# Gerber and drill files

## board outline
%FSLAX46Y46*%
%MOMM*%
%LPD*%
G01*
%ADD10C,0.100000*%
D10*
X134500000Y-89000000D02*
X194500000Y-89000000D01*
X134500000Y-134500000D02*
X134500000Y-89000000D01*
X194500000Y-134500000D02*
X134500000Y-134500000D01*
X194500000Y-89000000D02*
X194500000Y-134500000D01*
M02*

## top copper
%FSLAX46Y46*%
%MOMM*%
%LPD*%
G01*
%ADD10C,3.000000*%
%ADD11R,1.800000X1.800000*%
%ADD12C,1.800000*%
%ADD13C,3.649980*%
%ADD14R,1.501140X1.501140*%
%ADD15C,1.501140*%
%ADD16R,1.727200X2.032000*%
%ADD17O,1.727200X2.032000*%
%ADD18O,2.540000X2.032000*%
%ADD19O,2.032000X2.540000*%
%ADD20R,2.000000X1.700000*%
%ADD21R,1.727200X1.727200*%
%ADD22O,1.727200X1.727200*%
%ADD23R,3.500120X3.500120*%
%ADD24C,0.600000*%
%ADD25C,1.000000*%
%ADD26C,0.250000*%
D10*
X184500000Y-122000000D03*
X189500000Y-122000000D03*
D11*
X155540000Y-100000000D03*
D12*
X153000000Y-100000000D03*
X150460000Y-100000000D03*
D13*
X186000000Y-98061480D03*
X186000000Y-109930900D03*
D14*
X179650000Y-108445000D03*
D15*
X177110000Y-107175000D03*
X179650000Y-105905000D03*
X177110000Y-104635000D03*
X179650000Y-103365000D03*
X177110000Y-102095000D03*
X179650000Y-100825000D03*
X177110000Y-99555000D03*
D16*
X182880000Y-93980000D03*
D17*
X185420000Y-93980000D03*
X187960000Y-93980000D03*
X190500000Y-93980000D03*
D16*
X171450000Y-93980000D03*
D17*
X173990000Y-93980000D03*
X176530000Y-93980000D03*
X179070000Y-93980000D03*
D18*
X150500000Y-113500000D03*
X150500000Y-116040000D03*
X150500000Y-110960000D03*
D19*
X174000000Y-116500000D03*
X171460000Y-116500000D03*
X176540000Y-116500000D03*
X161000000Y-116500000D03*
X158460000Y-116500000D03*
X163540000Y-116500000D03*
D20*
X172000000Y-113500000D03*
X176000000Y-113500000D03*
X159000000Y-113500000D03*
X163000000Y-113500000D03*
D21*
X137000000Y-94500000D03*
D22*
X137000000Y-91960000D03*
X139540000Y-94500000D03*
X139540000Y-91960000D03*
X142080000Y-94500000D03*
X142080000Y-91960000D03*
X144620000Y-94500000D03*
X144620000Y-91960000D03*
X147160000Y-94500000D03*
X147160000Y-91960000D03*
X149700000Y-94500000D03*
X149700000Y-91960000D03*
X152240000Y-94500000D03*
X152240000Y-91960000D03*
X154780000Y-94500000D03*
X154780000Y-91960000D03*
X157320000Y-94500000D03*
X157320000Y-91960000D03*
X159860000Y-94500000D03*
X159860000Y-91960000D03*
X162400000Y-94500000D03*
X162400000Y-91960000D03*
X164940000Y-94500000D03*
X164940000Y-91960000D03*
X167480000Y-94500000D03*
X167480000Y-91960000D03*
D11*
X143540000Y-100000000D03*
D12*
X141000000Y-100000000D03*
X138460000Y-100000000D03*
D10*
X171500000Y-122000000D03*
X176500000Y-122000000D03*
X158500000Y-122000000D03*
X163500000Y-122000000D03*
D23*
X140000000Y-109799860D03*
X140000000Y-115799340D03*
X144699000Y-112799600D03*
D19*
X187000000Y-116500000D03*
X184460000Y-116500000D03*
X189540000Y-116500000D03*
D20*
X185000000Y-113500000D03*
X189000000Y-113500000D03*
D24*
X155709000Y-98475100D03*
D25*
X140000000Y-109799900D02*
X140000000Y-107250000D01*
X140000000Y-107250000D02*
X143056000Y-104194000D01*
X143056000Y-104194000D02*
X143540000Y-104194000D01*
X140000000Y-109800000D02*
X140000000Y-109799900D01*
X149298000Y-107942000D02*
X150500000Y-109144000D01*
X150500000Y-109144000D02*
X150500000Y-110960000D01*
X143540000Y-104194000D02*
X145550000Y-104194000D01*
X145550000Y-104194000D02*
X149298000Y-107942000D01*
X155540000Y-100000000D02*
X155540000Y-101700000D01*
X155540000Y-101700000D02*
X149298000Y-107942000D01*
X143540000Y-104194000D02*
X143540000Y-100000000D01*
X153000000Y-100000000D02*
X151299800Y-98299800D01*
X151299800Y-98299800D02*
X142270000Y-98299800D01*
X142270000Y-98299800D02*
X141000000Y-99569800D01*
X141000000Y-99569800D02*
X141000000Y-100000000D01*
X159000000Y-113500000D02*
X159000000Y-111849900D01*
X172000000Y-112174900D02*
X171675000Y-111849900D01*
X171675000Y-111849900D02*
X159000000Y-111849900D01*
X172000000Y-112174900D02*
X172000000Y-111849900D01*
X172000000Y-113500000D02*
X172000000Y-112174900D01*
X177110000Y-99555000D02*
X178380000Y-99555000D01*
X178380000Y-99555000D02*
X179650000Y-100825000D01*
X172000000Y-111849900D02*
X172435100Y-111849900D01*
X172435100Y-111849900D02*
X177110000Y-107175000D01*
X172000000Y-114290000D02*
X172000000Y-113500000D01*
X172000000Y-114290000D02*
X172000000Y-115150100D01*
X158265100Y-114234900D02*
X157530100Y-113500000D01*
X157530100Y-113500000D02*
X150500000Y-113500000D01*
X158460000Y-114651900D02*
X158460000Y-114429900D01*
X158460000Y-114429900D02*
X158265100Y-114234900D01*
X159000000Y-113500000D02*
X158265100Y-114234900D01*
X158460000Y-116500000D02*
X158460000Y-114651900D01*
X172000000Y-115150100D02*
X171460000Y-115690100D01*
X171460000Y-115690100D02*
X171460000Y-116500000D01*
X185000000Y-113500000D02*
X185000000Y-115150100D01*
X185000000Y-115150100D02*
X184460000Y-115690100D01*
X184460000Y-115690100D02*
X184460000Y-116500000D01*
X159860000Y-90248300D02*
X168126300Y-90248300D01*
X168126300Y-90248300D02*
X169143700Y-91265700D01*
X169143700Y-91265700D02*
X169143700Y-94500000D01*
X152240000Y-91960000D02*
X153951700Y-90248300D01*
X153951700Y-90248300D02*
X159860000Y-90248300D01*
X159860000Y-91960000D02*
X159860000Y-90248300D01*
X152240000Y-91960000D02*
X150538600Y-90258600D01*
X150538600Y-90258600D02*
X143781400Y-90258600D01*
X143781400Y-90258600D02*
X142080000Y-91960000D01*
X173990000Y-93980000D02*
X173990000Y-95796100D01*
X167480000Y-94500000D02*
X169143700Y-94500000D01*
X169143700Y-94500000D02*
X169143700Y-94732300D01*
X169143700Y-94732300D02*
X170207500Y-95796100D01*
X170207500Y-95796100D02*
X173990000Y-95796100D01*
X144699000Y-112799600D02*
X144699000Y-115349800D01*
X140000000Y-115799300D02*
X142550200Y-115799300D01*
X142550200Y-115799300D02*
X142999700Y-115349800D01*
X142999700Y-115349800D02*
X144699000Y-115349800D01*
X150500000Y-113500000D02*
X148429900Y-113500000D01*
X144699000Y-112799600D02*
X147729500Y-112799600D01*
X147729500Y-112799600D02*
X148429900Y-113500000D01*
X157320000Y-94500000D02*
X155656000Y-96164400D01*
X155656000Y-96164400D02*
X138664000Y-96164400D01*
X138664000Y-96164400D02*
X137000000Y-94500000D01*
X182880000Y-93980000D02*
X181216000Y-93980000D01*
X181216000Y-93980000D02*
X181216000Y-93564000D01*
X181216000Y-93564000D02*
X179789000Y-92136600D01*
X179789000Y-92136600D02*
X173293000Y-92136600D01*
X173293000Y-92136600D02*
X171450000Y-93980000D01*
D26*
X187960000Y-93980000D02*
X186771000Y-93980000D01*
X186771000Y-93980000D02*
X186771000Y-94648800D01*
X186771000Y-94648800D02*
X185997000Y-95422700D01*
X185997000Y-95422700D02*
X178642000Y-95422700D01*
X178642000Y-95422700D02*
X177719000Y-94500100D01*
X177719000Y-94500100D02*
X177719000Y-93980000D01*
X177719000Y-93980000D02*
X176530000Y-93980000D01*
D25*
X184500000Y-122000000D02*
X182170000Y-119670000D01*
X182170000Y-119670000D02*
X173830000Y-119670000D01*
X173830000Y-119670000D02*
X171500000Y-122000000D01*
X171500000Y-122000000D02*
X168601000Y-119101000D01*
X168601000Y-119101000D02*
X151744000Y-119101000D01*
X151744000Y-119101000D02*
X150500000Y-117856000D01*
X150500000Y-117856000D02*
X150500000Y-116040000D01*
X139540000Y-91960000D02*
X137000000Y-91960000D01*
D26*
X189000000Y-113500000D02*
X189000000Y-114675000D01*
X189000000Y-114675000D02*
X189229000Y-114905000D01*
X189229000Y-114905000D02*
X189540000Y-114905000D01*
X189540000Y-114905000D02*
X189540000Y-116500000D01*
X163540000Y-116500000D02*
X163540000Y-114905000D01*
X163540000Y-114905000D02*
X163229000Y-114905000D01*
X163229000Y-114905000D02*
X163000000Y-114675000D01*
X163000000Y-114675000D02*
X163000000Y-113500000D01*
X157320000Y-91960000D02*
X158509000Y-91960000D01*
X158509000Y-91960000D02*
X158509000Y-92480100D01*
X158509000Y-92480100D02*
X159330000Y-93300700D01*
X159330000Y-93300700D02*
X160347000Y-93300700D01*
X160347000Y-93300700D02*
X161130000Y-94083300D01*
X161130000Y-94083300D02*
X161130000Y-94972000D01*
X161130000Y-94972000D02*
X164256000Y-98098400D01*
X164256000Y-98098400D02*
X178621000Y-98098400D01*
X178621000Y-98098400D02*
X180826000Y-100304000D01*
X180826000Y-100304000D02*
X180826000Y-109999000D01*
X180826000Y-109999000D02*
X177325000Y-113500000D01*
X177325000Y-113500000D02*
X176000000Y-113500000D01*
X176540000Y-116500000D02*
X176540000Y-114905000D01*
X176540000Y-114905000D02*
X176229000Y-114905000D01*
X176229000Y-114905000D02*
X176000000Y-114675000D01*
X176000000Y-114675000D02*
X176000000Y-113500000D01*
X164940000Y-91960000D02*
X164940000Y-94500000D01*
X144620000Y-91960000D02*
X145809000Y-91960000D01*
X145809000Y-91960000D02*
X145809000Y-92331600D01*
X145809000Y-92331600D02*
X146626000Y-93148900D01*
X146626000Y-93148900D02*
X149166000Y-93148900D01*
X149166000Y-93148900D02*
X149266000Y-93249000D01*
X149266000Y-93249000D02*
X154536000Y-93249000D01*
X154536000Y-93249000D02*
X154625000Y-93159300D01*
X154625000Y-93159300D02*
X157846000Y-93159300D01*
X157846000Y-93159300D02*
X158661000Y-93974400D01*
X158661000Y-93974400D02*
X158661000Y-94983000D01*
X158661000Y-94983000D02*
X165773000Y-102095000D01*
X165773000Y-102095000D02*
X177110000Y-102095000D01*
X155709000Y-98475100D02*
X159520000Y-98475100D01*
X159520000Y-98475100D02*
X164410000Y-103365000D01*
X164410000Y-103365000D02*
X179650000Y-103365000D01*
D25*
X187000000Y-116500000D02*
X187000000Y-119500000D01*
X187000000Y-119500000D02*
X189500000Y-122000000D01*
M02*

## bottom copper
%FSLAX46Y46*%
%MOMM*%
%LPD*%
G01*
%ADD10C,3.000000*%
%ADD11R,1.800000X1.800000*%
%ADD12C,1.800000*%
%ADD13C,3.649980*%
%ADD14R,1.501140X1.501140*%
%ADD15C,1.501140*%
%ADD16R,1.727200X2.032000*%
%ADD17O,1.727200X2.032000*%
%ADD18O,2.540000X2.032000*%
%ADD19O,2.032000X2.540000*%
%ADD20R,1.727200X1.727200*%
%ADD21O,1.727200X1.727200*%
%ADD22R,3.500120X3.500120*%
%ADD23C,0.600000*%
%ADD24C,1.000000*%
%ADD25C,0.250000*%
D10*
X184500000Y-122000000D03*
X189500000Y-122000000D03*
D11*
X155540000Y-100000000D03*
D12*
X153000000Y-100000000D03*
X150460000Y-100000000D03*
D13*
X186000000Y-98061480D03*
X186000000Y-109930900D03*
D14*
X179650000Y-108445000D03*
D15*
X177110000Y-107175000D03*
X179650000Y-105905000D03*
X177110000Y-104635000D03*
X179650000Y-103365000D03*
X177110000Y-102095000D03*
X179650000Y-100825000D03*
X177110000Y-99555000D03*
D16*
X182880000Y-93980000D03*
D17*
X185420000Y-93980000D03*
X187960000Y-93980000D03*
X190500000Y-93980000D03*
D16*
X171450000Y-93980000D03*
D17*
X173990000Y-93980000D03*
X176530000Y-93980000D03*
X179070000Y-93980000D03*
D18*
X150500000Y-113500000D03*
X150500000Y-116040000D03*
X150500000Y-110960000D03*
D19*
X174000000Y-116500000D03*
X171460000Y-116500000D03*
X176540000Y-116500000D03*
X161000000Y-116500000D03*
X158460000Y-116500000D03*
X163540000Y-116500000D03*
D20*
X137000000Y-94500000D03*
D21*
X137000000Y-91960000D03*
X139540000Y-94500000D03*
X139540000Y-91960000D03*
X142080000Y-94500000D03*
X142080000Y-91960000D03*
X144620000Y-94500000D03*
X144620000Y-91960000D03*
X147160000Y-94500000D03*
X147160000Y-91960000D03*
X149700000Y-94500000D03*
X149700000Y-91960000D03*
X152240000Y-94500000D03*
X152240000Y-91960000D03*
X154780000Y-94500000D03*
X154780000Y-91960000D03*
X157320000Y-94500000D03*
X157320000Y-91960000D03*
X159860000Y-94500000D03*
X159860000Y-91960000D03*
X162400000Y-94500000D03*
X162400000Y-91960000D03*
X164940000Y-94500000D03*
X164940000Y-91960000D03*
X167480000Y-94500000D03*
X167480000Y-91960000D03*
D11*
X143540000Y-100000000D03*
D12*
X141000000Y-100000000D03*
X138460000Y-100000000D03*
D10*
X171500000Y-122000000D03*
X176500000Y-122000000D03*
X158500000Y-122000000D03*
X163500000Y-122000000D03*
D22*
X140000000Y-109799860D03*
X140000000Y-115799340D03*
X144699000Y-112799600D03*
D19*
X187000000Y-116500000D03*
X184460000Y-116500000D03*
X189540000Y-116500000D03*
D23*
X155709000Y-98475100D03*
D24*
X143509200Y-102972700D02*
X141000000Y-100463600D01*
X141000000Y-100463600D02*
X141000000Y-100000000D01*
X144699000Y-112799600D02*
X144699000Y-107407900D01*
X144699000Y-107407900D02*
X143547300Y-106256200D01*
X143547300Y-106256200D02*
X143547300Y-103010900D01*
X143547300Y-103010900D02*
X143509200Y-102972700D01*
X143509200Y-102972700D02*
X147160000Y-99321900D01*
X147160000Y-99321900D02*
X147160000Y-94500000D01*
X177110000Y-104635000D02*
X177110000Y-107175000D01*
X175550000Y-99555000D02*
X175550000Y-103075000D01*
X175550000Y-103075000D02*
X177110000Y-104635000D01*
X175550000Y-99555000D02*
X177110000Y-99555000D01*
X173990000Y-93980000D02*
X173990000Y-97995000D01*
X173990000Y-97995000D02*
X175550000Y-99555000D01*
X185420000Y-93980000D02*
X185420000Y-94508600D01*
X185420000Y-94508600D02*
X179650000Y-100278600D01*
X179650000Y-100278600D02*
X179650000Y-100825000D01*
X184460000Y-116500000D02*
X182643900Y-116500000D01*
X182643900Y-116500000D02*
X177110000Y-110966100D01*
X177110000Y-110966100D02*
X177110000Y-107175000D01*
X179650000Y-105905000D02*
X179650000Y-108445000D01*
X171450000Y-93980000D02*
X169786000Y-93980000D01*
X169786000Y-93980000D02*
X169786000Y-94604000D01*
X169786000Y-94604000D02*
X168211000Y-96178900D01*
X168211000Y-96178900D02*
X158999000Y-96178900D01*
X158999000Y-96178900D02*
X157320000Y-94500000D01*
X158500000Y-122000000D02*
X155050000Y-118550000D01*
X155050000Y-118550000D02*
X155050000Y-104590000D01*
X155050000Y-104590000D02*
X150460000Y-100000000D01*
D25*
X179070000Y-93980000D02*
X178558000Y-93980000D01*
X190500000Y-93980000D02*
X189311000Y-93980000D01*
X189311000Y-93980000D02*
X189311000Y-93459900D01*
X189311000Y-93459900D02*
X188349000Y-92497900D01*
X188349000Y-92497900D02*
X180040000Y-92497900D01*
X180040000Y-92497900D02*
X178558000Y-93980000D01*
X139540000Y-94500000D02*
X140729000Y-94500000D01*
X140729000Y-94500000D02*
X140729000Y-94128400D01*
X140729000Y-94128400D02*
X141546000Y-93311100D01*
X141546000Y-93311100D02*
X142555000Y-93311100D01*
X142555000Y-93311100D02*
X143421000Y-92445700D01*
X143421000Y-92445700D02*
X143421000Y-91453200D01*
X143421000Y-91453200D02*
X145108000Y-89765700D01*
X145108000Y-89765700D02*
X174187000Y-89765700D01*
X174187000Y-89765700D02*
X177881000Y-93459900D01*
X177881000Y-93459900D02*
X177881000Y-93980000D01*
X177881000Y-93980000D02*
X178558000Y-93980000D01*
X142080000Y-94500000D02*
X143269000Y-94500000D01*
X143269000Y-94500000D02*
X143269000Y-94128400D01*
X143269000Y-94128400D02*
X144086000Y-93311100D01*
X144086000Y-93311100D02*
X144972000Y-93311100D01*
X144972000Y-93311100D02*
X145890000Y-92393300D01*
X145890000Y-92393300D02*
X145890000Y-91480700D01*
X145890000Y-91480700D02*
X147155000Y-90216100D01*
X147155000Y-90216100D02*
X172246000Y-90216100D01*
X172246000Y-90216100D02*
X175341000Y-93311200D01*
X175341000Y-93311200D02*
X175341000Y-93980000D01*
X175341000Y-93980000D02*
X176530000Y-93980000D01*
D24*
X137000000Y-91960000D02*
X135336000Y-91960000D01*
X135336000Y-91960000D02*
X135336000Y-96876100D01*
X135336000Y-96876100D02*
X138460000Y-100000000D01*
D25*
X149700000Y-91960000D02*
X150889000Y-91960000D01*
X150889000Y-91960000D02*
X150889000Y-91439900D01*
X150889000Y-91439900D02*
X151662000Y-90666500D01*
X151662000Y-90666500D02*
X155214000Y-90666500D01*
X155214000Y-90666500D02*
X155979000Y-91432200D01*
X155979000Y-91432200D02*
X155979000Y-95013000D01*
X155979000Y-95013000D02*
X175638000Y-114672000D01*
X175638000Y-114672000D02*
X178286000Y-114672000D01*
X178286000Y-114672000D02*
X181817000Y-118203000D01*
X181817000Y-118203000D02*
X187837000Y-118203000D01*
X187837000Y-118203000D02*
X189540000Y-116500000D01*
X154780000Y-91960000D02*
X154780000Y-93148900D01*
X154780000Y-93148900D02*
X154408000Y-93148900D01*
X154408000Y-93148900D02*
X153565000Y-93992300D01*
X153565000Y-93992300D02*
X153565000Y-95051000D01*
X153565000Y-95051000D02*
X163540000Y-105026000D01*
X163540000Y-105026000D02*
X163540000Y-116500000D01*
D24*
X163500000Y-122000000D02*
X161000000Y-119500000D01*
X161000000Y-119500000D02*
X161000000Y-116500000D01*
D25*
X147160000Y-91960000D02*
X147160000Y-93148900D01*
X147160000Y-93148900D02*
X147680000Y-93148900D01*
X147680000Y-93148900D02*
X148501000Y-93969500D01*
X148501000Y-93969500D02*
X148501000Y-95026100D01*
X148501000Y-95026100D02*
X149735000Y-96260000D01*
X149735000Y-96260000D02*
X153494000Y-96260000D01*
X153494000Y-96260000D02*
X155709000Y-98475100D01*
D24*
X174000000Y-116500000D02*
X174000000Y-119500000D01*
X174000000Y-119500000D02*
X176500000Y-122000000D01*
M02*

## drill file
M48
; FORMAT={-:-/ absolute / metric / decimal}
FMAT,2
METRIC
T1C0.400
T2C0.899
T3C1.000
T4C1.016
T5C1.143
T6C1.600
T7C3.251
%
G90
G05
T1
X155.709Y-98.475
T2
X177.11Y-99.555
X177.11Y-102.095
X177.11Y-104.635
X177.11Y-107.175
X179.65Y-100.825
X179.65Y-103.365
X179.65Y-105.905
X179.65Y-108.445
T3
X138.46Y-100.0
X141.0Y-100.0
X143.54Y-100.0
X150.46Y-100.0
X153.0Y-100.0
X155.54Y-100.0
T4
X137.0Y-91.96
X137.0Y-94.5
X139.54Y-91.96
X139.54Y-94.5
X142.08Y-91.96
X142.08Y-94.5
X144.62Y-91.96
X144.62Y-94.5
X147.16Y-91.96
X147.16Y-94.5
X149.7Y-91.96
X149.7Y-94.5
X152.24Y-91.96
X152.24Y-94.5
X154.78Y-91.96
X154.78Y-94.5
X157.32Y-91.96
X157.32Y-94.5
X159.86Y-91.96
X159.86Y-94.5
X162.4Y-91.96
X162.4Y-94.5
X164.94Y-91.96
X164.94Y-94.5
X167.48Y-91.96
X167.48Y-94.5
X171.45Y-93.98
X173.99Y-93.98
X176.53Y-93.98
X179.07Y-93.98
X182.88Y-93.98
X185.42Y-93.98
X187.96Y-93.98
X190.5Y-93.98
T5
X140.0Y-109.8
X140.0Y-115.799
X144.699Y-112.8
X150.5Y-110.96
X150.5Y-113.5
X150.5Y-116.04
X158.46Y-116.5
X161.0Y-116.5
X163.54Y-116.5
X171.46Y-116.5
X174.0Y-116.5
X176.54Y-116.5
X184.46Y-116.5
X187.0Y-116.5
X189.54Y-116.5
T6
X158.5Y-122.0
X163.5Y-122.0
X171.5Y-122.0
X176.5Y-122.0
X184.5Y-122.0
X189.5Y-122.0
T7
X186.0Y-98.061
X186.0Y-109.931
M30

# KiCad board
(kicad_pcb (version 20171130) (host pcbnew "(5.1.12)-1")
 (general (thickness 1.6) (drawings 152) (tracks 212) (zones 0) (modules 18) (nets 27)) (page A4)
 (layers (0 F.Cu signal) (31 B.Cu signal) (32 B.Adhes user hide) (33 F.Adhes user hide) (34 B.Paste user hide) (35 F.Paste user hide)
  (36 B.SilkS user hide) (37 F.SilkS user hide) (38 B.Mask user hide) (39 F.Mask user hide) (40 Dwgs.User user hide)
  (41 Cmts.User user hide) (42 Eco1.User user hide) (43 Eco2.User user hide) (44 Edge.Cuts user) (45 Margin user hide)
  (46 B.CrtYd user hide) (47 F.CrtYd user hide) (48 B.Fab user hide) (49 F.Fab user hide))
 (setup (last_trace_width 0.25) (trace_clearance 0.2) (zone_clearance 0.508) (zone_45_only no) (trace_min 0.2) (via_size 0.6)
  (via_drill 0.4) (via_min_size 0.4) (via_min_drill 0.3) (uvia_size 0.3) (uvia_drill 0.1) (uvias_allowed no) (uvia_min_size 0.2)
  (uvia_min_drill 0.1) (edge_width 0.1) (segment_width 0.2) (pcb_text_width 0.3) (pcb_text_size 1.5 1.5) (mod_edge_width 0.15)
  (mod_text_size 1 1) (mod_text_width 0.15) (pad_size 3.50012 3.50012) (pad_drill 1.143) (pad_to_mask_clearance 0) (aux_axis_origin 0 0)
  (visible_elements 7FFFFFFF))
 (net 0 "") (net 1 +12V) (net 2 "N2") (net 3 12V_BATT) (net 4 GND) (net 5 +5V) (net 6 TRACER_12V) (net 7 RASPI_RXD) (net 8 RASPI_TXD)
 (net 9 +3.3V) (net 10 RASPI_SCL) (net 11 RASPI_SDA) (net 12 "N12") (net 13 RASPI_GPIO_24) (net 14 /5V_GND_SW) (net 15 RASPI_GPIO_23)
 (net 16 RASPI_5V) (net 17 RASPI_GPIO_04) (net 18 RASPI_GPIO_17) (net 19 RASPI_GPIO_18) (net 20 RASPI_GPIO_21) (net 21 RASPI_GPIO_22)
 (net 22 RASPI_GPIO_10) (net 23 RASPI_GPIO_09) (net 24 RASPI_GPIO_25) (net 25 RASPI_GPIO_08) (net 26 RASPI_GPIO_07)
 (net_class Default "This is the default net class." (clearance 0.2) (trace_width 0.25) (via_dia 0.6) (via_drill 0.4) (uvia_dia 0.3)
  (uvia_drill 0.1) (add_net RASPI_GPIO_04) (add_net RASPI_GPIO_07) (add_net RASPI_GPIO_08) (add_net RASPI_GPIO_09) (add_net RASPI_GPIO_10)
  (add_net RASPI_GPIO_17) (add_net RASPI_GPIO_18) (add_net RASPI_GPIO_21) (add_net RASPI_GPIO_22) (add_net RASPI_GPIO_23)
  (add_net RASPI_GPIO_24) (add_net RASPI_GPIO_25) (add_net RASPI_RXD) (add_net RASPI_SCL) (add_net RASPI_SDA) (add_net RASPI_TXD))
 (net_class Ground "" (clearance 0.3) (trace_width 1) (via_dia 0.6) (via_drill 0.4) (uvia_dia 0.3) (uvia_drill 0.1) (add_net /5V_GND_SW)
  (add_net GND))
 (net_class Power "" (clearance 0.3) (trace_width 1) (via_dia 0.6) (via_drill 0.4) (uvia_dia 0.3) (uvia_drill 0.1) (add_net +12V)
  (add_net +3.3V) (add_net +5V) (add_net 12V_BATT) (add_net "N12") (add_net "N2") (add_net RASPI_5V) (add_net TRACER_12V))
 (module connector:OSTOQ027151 (layer F.Cu) (at 187 126)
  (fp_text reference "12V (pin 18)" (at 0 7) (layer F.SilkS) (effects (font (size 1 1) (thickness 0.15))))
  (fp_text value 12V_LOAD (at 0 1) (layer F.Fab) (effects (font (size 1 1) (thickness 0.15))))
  (pad 1 thru_hole circle (at -2.5 -4) (size 3 3) (drill 1.6) (layers *.Cu *.Mask F.SilkS) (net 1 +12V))
  (pad 2 thru_hole circle (at 2.5 -4) (size 3 3) (drill 1.6) (layers *.Cu *.Mask F.SilkS) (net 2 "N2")))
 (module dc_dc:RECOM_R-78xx (layer F.Cu) (at 153 100 180)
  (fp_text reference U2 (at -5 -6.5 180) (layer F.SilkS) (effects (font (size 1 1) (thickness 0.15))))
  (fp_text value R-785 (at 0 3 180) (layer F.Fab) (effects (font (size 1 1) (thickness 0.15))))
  (pad 1 thru_hole rect (at -2.54 0 270) (size 1.8 1.8) (drill 1) (layers *.Cu *.Mask F.SilkS) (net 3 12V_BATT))
  (pad 2 thru_hole circle (at 0 0 270) (size 1.8 1.8) (drill 1) (layers *.Cu *.Mask F.SilkS) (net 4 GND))
  (pad 3 thru_hole circle (at 2.54 0 270) (size 1.8 1.8) (drill 1) (layers *.Cu *.Mask F.SilkS) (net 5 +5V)))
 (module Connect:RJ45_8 (layer F.Cu) (at 186 104 90)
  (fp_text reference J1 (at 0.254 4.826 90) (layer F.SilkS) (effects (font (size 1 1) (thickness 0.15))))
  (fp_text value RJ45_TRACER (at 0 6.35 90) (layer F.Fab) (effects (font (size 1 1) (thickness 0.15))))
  (pad Hole np_thru_hole circle (at 5.93852 0 90) (size 3.64998 3.64998) (drill 3.2512) (layers *.Cu *.SilkS *.Mask))
  (pad Hole np_thru_hole circle (at -5.9309 0 90) (size 3.64998 3.64998) (drill 3.2512) (layers *.Cu *.SilkS *.Mask))
  (pad 1 thru_hole rect (at -4.445 -6.35 90) (size 1.50114 1.50114) (drill 0.89916) (layers *.Cu *.Mask F.SilkS) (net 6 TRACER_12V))
  (pad 2 thru_hole circle (at -3.175 -8.89 90) (size 1.50114 1.50114) (drill 0.89916) (layers *.Cu *.Mask F.SilkS) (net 4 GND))
  (pad 3 thru_hole circle (at -1.905 -6.35 90) (size 1.50114 1.50114) (drill 0.89916) (layers *.Cu *.Mask F.SilkS) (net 6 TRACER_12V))
  (pad 4 thru_hole circle (at -0.635 -8.89 90) (size 1.50114 1.50114) (drill 0.89916) (layers *.Cu *.Mask F.SilkS) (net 4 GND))
  (pad 5 thru_hole circle (at 0.635 -6.35 90) (size 1.50114 1.50114) (drill 0.89916) (layers *.Cu *.Mask F.SilkS) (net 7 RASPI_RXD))
  (pad 6 thru_hole circle (at 1.905 -8.89 90) (size 1.50114 1.50114) (drill 0.89916) (layers *.Cu *.Mask F.SilkS) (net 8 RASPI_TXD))
  (pad 7 thru_hole circle (at 3.175 -6.35 90) (size 1.50114 1.50114) (drill 0.89916) (layers *.Cu *.Mask F.SilkS) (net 4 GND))
  (pad 8 thru_hole circle (at 4.445 -8.89 90) (size 1.50114 1.50114) (drill 0.89916) (layers *.Cu *.Mask F.SilkS) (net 4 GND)))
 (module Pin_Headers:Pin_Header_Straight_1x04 (layer F.Cu) (at 182.88 93.98 90)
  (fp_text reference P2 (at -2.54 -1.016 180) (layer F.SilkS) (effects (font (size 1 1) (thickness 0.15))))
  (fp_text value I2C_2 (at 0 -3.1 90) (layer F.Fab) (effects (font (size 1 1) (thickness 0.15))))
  (pad 1 thru_hole rect (at 0 0 90) (size 2.032 1.7272) (drill 1.016) (layers *.Cu *.Mask F.SilkS) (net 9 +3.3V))
  (pad 2 thru_hole oval (at 0 2.54 90) (size 2.032 1.7272) (drill 1.016) (layers *.Cu *.Mask F.SilkS) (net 4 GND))
  (pad 3 thru_hole oval (at 0 5.08 90) (size 2.032 1.7272) (drill 1.016) (layers *.Cu *.Mask F.SilkS) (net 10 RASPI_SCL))
  (pad 4 thru_hole oval (at 0 7.62 90) (size 2.032 1.7272) (drill 1.016) (layers *.Cu *.Mask F.SilkS) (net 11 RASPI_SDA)))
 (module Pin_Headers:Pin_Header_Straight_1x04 (layer F.Cu) (at 171.45 93.98 90)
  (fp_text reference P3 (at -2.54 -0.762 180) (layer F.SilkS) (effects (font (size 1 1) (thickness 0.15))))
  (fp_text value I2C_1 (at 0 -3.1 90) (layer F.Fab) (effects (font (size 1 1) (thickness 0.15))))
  (pad 1 thru_hole rect (at 0 0 90) (size 2.032 1.7272) (drill 1.016) (layers *.Cu *.Mask F.SilkS) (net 9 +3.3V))
  (pad 2 thru_hole oval (at 0 2.54 90) (size 2.032 1.7272) (drill 1.016) (layers *.Cu *.Mask F.SilkS) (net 4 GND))
  (pad 3 thru_hole oval (at 0 5.08 90) (size 2.032 1.7272) (drill 1.016) (layers *.Cu *.Mask F.SilkS) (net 10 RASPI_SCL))
  (pad 4 thru_hole oval (at 0 7.62 90) (size 2.032 1.7272) (drill 1.016) (layers *.Cu *.Mask F.SilkS) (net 11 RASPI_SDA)))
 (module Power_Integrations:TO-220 (layer F.Cu) (at 150.5 113.5 270)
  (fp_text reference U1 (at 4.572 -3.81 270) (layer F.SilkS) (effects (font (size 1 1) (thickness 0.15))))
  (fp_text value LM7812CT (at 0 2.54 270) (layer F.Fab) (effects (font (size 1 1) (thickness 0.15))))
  (pad 2 thru_hole oval (at 0 0 270) (size 2.032 2.54) (drill 1.143) (layers *.Cu *.Mask F.SilkS) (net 4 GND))
  (pad 3 thru_hole oval (at 2.54 0 270) (size 2.032 2.54) (drill 1.143) (layers *.Cu *.Mask F.SilkS) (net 1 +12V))
  (pad 1 thru_hole oval (at -2.54 0 270) (size 2.032 2.54) (drill 1.143) (layers *.Cu *.Mask F.SilkS) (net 3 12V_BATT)))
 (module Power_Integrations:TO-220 (layer F.Cu) (at 174 116.5 180)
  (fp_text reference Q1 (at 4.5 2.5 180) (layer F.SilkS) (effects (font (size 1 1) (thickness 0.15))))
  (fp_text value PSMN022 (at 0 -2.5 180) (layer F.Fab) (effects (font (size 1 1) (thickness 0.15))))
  (pad 2 thru_hole oval (at 0 0 180) (size 2.032 2.54) (drill 1.143) (layers *.Cu *.Mask F.SilkS) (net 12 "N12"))
  (pad 3 thru_hole oval (at 2.54 0 180) (size 2.032 2.54) (drill 1.143) (layers *.Cu *.Mask F.SilkS) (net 4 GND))
  (pad 1 thru_hole oval (at -2.54 0 180) (size 2.032 2.54) (drill 1.143) (layers *.Cu *.Mask F.SilkS) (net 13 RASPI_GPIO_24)))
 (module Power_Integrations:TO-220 (layer F.Cu) (at 161 116.5 180)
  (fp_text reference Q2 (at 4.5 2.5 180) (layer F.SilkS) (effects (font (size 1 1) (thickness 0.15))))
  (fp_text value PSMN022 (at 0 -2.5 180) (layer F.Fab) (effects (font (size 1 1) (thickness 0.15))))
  (pad 2 thru_hole oval (at 0 0 180) (size 2.032 2.54) (drill 1.143) (layers *.Cu *.Mask F.SilkS) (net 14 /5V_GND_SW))
  (pad 3 thru_hole oval (at 2.54 0 180) (size 2.032 2.54) (drill 1.143) (layers *.Cu *.Mask F.SilkS) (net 4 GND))
  (pad 1 thru_hole oval (at -2.54 0 180) (size 2.032 2.54) (drill 1.143) (layers *.Cu *.Mask F.SilkS) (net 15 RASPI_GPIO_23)))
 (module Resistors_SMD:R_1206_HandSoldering (layer F.Cu) (at 174 113.5)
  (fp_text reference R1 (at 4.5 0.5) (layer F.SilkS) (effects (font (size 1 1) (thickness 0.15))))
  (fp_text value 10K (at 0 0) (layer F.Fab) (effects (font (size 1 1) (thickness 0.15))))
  (pad 1 smd rect (at -2 0) (size 2 1.7) (layers F.Cu F.Paste F.Mask) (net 4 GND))
  (pad 2 smd rect (at 2 0) (size 2 1.7) (layers F.Cu F.Paste F.Mask) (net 13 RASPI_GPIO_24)))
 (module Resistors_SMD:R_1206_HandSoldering (layer F.Cu) (at 161 113.5)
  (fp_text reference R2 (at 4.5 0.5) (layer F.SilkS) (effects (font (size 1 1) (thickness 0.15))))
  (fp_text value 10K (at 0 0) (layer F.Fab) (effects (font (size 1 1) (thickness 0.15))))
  (pad 1 smd rect (at -2 0) (size 2 1.7) (layers F.Cu F.Paste F.Mask) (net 4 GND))
  (pad 2 smd rect (at 2 0) (size 2 1.7) (layers F.Cu F.Paste F.Mask) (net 15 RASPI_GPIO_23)))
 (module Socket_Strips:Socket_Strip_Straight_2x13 (layer B.Cu) (at 137 94.5)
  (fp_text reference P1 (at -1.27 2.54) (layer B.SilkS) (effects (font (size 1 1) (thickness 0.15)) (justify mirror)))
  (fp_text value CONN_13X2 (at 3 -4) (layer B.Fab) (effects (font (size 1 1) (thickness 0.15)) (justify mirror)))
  (pad 1 thru_hole rect (at 0 0) (size 1.7272 1.7272) (drill 1.016) (layers *.Cu *.Mask B.SilkS) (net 9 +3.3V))
  (pad 2 thru_hole oval (at 0 -2.54) (size 1.7272 1.7272) (drill 1.016) (layers *.Cu *.Mask B.SilkS) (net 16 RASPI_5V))
  (pad 3 thru_hole oval (at 2.54 0) (size 1.7272 1.7272) (drill 1.016) (layers *.Cu *.Mask B.SilkS) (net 11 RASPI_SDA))
  (pad 4 thru_hole oval (at 2.54 -2.54) (size 1.7272 1.7272) (drill 1.016) (layers *.Cu *.Mask B.SilkS) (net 16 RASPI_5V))
  (pad 5 thru_hole oval (at 5.08 0) (size 1.7272 1.7272) (drill 1.016) (layers *.Cu *.Mask B.SilkS) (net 10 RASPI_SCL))
  (pad 6 thru_hole oval (at 5.08 -2.54) (size 1.7272 1.7272) (drill 1.016) (layers *.Cu *.Mask B.SilkS) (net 4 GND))
  (pad 7 thru_hole oval (at 7.62 0) (size 1.7272 1.7272) (drill 1.016) (layers *.Cu *.Mask B.SilkS) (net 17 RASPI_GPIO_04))
  (pad 8 thru_hole oval (at 7.62 -2.54) (size 1.7272 1.7272) (drill 1.016) (layers *.Cu *.Mask B.SilkS) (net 8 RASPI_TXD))
  (pad 9 thru_hole oval (at 10.16 0) (size 1.7272 1.7272) (drill 1.016) (layers *.Cu *.Mask B.SilkS) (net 4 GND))
  (pad 10 thru_hole oval (at 10.16 -2.54) (size 1.7272 1.7272) (drill 1.016) (layers *.Cu *.Mask B.SilkS) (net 7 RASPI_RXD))
  (pad 11 thru_hole oval (at 12.7 0) (size 1.7272 1.7272) (drill 1.016) (layers *.Cu *.Mask B.SilkS) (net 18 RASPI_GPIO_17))
  (pad 12 thru_hole oval (at 12.7 -2.54) (size 1.7272 1.7272) (drill 1.016) (layers *.Cu *.Mask B.SilkS) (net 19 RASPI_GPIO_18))
  (pad 13 thru_hole oval (at 15.24 0) (size 1.7272 1.7272) (drill 1.016) (layers *.Cu *.Mask B.SilkS) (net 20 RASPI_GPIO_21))
  (pad 14 thru_hole oval (at 15.24 -2.54) (size 1.7272 1.7272) (drill 1.016) (layers *.Cu *.Mask B.SilkS) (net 4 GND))
  (pad 15 thru_hole oval (at 17.78 0) (size 1.7272 1.7272) (drill 1.016) (layers *.Cu *.Mask B.SilkS) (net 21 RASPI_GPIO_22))
  (pad 16 thru_hole oval (at 17.78 -2.54) (size 1.7272 1.7272) (drill 1.016) (layers *.Cu *.Mask B.SilkS) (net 15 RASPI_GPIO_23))
  (pad 17 thru_hole oval (at 20.32 0) (size 1.7272 1.7272) (drill 1.016) (layers *.Cu *.Mask B.SilkS) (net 9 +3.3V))
  (pad 18 thru_hole oval (at 20.32 -2.54) (size 1.7272 1.7272) (drill 1.016) (layers *.Cu *.Mask B.SilkS) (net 13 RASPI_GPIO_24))
  (pad 19 thru_hole oval (at 22.86 0) (size 1.7272 1.7272) (drill 1.016) (layers *.Cu *.Mask B.SilkS) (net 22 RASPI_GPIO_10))
  (pad 20 thru_hole oval (at 22.86 -2.54) (size 1.7272 1.7272) (drill 1.016) (layers *.Cu *.Mask B.SilkS) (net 4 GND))
  (pad 21 thru_hole oval (at 25.4 0) (size 1.7272 1.7272) (drill 1.016) (layers *.Cu *.Mask B.SilkS) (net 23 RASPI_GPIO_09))
  (pad 22 thru_hole oval (at 25.4 -2.54) (size 1.7272 1.7272) (drill 1.016) (layers *.Cu *.Mask B.SilkS) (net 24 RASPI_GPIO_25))
  (pad 23 thru_hole oval (at 27.94 0) (size 1.7272 1.7272) (drill 1.016) (layers *.Cu *.Mask B.SilkS) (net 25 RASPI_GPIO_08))
  (pad 24 thru_hole oval (at 27.94 -2.54) (size 1.7272 1.7272) (drill 1.016) (layers *.Cu *.Mask B.SilkS) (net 25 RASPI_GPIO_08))
  (pad 25 thru_hole oval (at 30.48 0) (size 1.7272 1.7272) (drill 1.016) (layers *.Cu *.Mask B.SilkS) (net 4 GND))
  (pad 26 thru_hole oval (at 30.48 -2.54) (size 1.7272 1.7272) (drill 1.016) (layers *.Cu *.Mask B.SilkS) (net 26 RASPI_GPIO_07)))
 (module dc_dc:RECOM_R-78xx (layer F.Cu) (at 141 100 180)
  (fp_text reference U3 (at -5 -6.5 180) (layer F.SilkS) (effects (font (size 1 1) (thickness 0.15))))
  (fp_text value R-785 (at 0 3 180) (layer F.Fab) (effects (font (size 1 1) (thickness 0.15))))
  (pad 1 thru_hole rect (at -2.54 0 270) (size 1.8 1.8) (drill 1) (layers *.Cu *.Mask F.SilkS) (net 3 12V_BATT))
  (pad 2 thru_hole circle (at 0 0 270) (size 1.8 1.8) (drill 1) (layers *.Cu *.Mask F.SilkS) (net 4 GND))
  (pad 3 thru_hole circle (at 2.54 0 270) (size 1.8 1.8) (drill 1) (layers *.Cu *.Mask F.SilkS) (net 16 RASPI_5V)))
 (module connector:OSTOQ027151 (layer F.Cu) (at 174 126)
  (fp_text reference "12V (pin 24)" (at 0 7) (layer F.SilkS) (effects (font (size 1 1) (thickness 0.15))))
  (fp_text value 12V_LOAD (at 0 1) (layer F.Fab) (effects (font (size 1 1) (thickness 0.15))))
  (pad 1 thru_hole circle (at -2.5 -4) (size 3 3) (drill 1.6) (layers *.Cu *.Mask F.SilkS) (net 1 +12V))
  (pad 2 thru_hole circle (at 2.5 -4) (size 3 3) (drill 1.6) (layers *.Cu *.Mask F.SilkS) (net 12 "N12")))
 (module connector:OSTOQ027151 (layer F.Cu) (at 161 126)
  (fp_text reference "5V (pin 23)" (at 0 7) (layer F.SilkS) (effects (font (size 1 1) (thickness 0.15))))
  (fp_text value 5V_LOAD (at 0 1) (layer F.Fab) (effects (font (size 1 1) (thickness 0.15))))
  (pad 1 thru_hole circle (at -2.5 -4) (size 3 3) (drill 1.6) (layers *.Cu *.Mask F.SilkS) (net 5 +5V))
  (pad 2 thru_hole circle (at 2.5 -4) (size 3 3) (drill 1.6) (layers *.Cu *.Mask F.SilkS) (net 14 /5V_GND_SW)))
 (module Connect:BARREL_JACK (layer F.Cu) (at 140 116 90)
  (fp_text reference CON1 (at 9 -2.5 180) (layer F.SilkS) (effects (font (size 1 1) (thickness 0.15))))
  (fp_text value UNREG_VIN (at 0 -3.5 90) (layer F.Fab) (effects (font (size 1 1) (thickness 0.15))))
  (pad 1 thru_hole rect (at 6.20014 0 90) (size 3.50012 3.50012) (drill 1.143) (layers *.Cu *.Mask F.SilkS) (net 3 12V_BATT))
  (pad 2 thru_hole rect (at 0.20066 0 90) (size 3.50012 3.50012) (drill 1.143) (layers *.Cu *.Mask F.SilkS) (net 4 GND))
  (pad 3 thru_hole rect (at 3.2004 4.699 90) (size 3.50012 3.50012) (drill 1.143) (layers *.Cu *.Mask F.SilkS) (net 4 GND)))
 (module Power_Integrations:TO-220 (layer F.Cu) (at 187 116.5 180)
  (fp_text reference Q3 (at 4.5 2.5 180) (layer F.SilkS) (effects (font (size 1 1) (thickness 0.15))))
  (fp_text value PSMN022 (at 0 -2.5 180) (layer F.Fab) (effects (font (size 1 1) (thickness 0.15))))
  (pad 2 thru_hole oval (at 0 0 180) (size 2.032 2.54) (drill 1.143) (layers *.Cu *.Mask F.SilkS) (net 2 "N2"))
  (pad 3 thru_hole oval (at 2.54 0 180) (size 2.032 2.54) (drill 1.143) (layers *.Cu *.Mask F.SilkS) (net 4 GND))
  (pad 1 thru_hole oval (at -2.54 0 180) (size 2.032 2.54) (drill 1.143) (layers *.Cu *.Mask F.SilkS) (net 19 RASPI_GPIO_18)))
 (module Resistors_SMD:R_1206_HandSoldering (layer F.Cu) (at 187 113.5)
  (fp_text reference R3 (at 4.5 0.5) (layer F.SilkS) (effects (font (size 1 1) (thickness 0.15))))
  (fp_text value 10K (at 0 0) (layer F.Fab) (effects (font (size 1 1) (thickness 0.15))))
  (pad 1 smd rect (at -2 0) (size 2 1.7) (layers F.Cu F.Paste F.Mask) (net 4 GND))
  (pad 2 smd rect (at 2 0) (size 2 1.7) (layers F.Cu F.Paste F.Mask) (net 19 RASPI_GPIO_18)))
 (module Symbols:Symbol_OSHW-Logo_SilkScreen (layer F.Cu) (at 150 125)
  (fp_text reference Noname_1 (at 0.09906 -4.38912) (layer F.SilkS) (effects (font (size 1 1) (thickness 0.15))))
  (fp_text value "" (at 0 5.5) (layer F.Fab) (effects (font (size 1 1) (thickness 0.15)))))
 (gr_line (start 134.5 89) (end 194.5 89) (angle 90) (layer Edge.Cuts) (width 0.1))
 (gr_line (start 134.5 134.5) (end 134.5 89) (angle 90) (layer Edge.Cuts) (width 0.1))
 (gr_line (start 194.5 134.5) (end 134.5 134.5) (angle 90) (layer Edge.Cuts) (width 0.1))
 (gr_line (start 194.5 89) (end 194.5 134.5) (angle 90) (layer Edge.Cuts) (width 0.1))
 (segment (start 140 109.7999) (end 140 107.25) (width 1) (layer F.Cu) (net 3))
 (segment (start 140 107.25) (end 143.056 104.194) (width 1) (layer F.Cu) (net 3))
 (segment (start 143.056 104.194) (end 143.54 104.194) (width 1) (layer F.Cu) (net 3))
 (segment (start 140 109.8) (end 140 109.7999) (width 1) (layer F.Cu) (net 3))
 (segment (start 149.298 107.942) (end 150.5 109.144) (width 1) (layer F.Cu) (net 3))
 (segment (start 150.5 109.144) (end 150.5 110.96) (width 1) (layer F.Cu) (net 3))
 (segment (start 143.54 104.194) (end 145.55 104.194) (width 1) (layer F.Cu) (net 3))
 (segment (start 145.55 104.194) (end 149.298 107.942) (width 1) (layer F.Cu) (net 3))
 (segment (start 155.54 100) (end 155.54 101.7) (width 1) (layer F.Cu) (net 3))
 (segment (start 155.54 101.7) (end 149.298 107.942) (width 1) (layer F.Cu) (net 3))
 (segment (start 143.54 104.194) (end 143.54 100) (width 1) (layer F.Cu) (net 3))
 (segment (start 153 100) (end 151.2998 98.2998) (width 1) (layer F.Cu) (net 4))
 (segment (start 151.2998 98.2998) (end 142.27 98.2998) (width 1) (layer F.Cu) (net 4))
 (segment (start 142.27 98.2998) (end 141 99.5698) (width 1) (layer F.Cu) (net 4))
 (segment (start 141 99.5698) (end 141 100) (width 1) (layer F.Cu) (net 4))
 (segment (start 143.5092 102.9727) (end 141 100.4636) (width 1) (layer B.Cu) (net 4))
 (segment (start 141 100.4636) (end 141 100) (width 1) (layer B.Cu) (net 4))
 (segment (start 144.699 112.7996) (end 144.699 107.4079) (width 1) (layer B.Cu) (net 4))
 (segment (start 144.699 107.4079) (end 143.5473 106.2562) (width 1) (layer B.Cu) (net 4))
 (segment (start 143.5473 106.2562) (end 143.5473 103.0109) (width 1) (layer B.Cu) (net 4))
 (segment (start 143.5473 103.0109) (end 143.5092 102.9727) (width 1) (layer B.Cu) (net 4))
 (segment (start 143.5092 102.9727) (end 147.16 99.3219) (width 1) (layer B.Cu) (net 4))
 (segment (start 147.16 99.3219) (end 147.16 94.5) (width 1) (layer B.Cu) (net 4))
 (segment (start 159 113.5) (end 159 111.8499) (width 1) (layer F.Cu) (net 4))
 (segment (start 172 112.1749) (end 171.675 111.8499) (width 1) (layer F.Cu) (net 4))
 (segment (start 171.675 111.8499) (end 159 111.8499) (width 1) (layer F.Cu) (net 4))
 (segment (start 172 112.1749) (end 172 111.8499) (width 1) (layer F.Cu) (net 4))
 (segment (start 172 113.5) (end 172 112.1749) (width 1) (layer F.Cu) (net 4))
 (segment (start 177.11 104.635) (end 177.11 107.175) (width 1) (layer B.Cu) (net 4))
 (segment (start 175.55 99.555) (end 175.55 103.075) (width 1) (layer B.Cu) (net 4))
 (segment (start 175.55 103.075) (end 177.11 104.635) (width 1) (layer B.Cu) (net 4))
 (segment (start 175.55 99.555) (end 177.11 99.555) (width 1) (layer B.Cu) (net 4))
 (segment (start 173.99 93.98) (end 173.99 97.995) (width 1) (layer B.Cu) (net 4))
 (segment (start 173.99 97.995) (end 175.55 99.555) (width 1) (layer B.Cu) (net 4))
 (segment (start 177.11 99.555) (end 178.38 99.555) (width 1) (layer F.Cu) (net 4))
 (segment (start 178.38 99.555) (end 179.65 100.825) (width 1) (layer F.Cu) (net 4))
 (segment (start 185.42 93.98) (end 185.42 94.5086) (width 1) (layer B.Cu) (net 4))
 (segment (start 185.42 94.5086) (end 179.65 100.2786) (width 1) (layer B.Cu) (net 4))
 (segment (start 179.65 100.2786) (end 179.65 100.825) (width 1) (layer B.Cu) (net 4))
 (segment (start 172 111.8499) (end 172.4351 111.8499) (width 1) (layer F.Cu) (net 4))
 (segment (start 172.4351 111.8499) (end 177.11 107.175) (width 1) (layer F.Cu) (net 4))
 (segment (start 172 114.29) (end 172 113.5) (width 1) (layer F.Cu) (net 4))
 (segment (start 172 114.29) (end 172 115.1501) (width 1) (layer F.Cu) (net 4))
 (segment (start 158.2651 114.2349) (end 157.5301 113.5) (width 1) (layer F.Cu) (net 4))
 (segment (start 157.5301 113.5) (end 150.5 113.5) (width 1) (layer F.Cu) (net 4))
 (segment (start 158.46 114.6519) (end 158.46 114.4299) (width 1) (layer F.Cu) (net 4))
 (segment (start 158.46 114.4299) (end 158.2651 114.2349) (width 1) (layer F.Cu) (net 4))
 (segment (start 159 113.5) (end 158.2651 114.2349) (width 1) (layer F.Cu) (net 4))
 (segment (start 158.46 116.5) (end 158.46 114.6519) (width 1) (layer F.Cu) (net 4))
 (segment (start 184.46 116.5) (end 182.6439 116.5) (width 1) (layer B.Cu) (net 4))
 (segment (start 182.6439 116.5) (end 177.11 110.9661) (width 1) (layer B.Cu) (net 4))
 (segment (start 177.11 110.9661) (end 177.11 107.175) (width 1) (layer B.Cu) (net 4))
 (segment (start 172 115.1501) (end 171.46 115.6901) (width 1) (layer F.Cu) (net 4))
 (segment (start 171.46 115.6901) (end 171.46 116.5) (width 1) (layer F.Cu) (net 4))
 (segment (start 185 113.5) (end 185 115.1501) (width 1) (layer F.Cu) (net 4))
 (segment (start 185 115.1501) (end 184.46 115.6901) (width 1) (layer F.Cu) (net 4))
 (segment (start 184.46 115.6901) (end 184.46 116.5) (width 1) (layer F.Cu) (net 4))
 (segment (start 159.86 90.2483) (end 168.1263 90.2483) (width 1) (layer F.Cu) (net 4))
 (segment (start 168.1263 90.2483) (end 169.1437 91.2657) (width 1) (layer F.Cu) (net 4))
 (segment (start 169.1437 91.2657) (end 169.1437 94.5) (width 1) (layer F.Cu) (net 4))
 (segment (start 152.24 91.96) (end 153.9517 90.2483) (width 1) (layer F.Cu) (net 4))
 (segment (start 153.9517 90.2483) (end 159.86 90.2483) (width 1) (layer F.Cu) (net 4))
 (segment (start 159.86 91.96) (end 159.86 90.2483) (width 1) (layer F.Cu) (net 4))
 (segment (start 152.24 91.96) (end 150.5386 90.2586) (width 1) (layer F.Cu) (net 4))
 (segment (start 150.5386 90.2586) (end 143.7814 90.2586) (width 1) (layer F.Cu) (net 4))
 (segment (start 143.7814 90.2586) (end 142.08 91.96) (width 1) (layer F.Cu) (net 4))
 (segment (start 173.99 93.98) (end 173.99 95.7961) (width 1) (layer F.Cu) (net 4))
 (segment (start 167.48 94.5) (end 169.1437 94.5) (width 1) (layer F.Cu) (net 4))
 (segment (start 169.1437 94.5) (end 169.1437 94.7323) (width 1) (layer F.Cu) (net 4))
 (segment (start 169.1437 94.7323) (end 170.2075 95.7961) (width 1) (layer F.Cu) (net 4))
 (segment (start 170.2075 95.7961) (end 173.99 95.7961) (width 1) (layer F.Cu) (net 4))
 (segment (start 144.699 112.7996) (end 144.699 115.3498) (width 1) (layer F.Cu) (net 4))
 (segment (start 140 115.7993) (end 142.5502 115.7993) (width 1) (layer F.Cu) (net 4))
 (segment (start 142.5502 115.7993) (end 142.9997 115.3498) (width 1) (layer F.Cu) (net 4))
 (segment (start 142.9997 115.3498) (end 144.699 115.3498) (width 1) (layer F.Cu) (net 4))
 (segment (start 150.5 113.5) (end 148.4299 113.5) (width 1) (layer F.Cu) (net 4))
 (segment (start 144.699 112.7996) (end 147.7295 112.7996) (width 1) (layer F.Cu) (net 4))
 (segment (start 147.7295 112.7996) (end 148.4299 113.5) (width 1) (layer F.Cu) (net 4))
 (segment (start 179.65 105.905) (end 179.65 108.445) (width 1) (layer B.Cu) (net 6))
 (segment (start 157.32 94.5) (end 155.656 96.1644) (width 1) (layer F.Cu) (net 9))
 (segment (start 155.656 96.1644) (end 138.664 96.1644) (width 1) (layer F.Cu) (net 9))
 (segment (start 138.664 96.1644) (end 137 94.5) (width 1) (layer F.Cu) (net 9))
 (segment (start 171.45 93.98) (end 169.786 93.98) (width 1) (layer B.Cu) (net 9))
 (segment (start 169.786 93.98) (end 169.786 94.604) (width 1) (layer B.Cu) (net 9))
 (segment (start 169.786 94.604) (end 168.211 96.1789) (width 1) (layer B.Cu) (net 9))
 (segment (start 168.211 96.1789) (end 158.999 96.1789) (width 1) (layer B.Cu) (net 9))
 (segment (start 158.999 96.1789) (end 157.32 94.5) (width 1) (layer B.Cu) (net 9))
 (segment (start 182.88 93.98) (end 181.216 93.98) (width 1) (layer F.Cu) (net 9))
 (segment (start 181.216 93.98) (end 181.216 93.564) (width 1) (layer F.Cu) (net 9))
 (segment (start 181.216 93.564) (end 179.789 92.1366) (width 1) (layer F.Cu) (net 9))
 (segment (start 179.789 92.1366) (end 173.293 92.1366) (width 1) (layer F.Cu) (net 9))
 (segment (start 173.293 92.1366) (end 171.45 93.98) (width 1) (layer F.Cu) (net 9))
 (segment (start 158.5 122) (end 155.05 118.55) (width 1) (layer B.Cu) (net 5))
 (segment (start 155.05 118.55) (end 155.05 104.59) (width 1) (layer B.Cu) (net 5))
 (segment (start 155.05 104.59) (end 150.46 100) (width 1) (layer B.Cu) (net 5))
 (segment (start 179.07 93.98) (end 178.558 93.98) (width 0.25) (layer B.Cu) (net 11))
 (segment (start 190.5 93.98) (end 189.311 93.98) (width 0.25) (layer B.Cu) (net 11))
 (segment (start 189.311 93.98) (end 189.311 93.4599) (width 0.25) (layer B.Cu) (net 11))
 (segment (start 189.311 93.4599) (end 188.349 92.4979) (width 0.25) (layer B.Cu) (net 11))
 (segment (start 188.349 92.4979) (end 180.04 92.4979) (width 0.25) (layer B.Cu) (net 11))
 (segment (start 180.04 92.4979) (end 178.558 93.98) (width 0.25) (layer B.Cu) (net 11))
 (segment (start 139.54 94.5) (end 140.729 94.5) (width 0.25) (layer B.Cu) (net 11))
 (segment (start 140.729 94.5) (end 140.729 94.1284) (width 0.25) (layer B.Cu) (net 11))
 (segment (start 140.729 94.1284) (end 141.546 93.3111) (width 0.25) (layer B.Cu) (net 11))
 (segment (start 141.546 93.3111) (end 142.555 93.3111) (width 0.25) (layer B.Cu) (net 11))
 (segment (start 142.555 93.3111) (end 143.421 92.4457) (width 0.25) (layer B.Cu) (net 11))
 (segment (start 143.421 92.4457) (end 143.421 91.4532) (width 0.25) (layer B.Cu) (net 11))
 (segment (start 143.421 91.4532) (end 145.108 89.7657) (width 0.25) (layer B.Cu) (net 11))
 (segment (start 145.108 89.7657) (end 174.187 89.7657) (width 0.25) (layer B.Cu) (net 11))
 (segment (start 174.187 89.7657) (end 177.881 93.4599) (width 0.25) (layer B.Cu) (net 11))
 (segment (start 177.881 93.4599) (end 177.881 93.98) (width 0.25) (layer B.Cu) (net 11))
 (segment (start 177.881 93.98) (end 178.558 93.98) (width 0.25) (layer B.Cu) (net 11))
 (segment (start 142.08 94.5) (end 143.269 94.5) (width 0.25) (layer B.Cu) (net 10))
 (segment (start 143.269 94.5) (end 143.269 94.1284) (width 0.25) (layer B.Cu) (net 10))
 (segment (start 143.269 94.1284) (end 144.086 93.3111) (width 0.25) (layer B.Cu) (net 10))
 (segment (start 144.086 93.3111) (end 144.972 93.3111) (width 0.25) (layer B.Cu) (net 10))
 (segment (start 144.972 93.3111) (end 145.89 92.3933) (width 0.25) (layer B.Cu) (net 10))
 (segment (start 145.89 92.3933) (end 145.89 91.4807) (width 0.25) (layer B.Cu) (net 10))
 (segment (start 145.89 91.4807) (end 147.155 90.2161) (width 0.25) (layer B.Cu) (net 10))
 (segment (start 147.155 90.2161) (end 172.246 90.2161) (width 0.25) (layer B.Cu) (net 10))
 (segment (start 172.246 90.2161) (end 175.341 93.3112) (width 0.25) (layer B.Cu) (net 10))
 (segment (start 175.341 93.3112) (end 175.341 93.98) (width 0.25) (layer B.Cu) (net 10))
 (segment (start 175.341 93.98) (end 176.53 93.98) (width 0.25) (layer B.Cu) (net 10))
 (segment (start 187.96 93.98) (end 186.771 93.98) (width 0.25) (layer F.Cu) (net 10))
 (segment (start 186.771 93.98) (end 186.771 94.6488) (width 0.25) (layer F.Cu) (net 10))
 (segment (start 186.771 94.6488) (end 185.997 95.4227) (width 0.25) (layer F.Cu) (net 10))
 (segment (start 185.997 95.4227) (end 178.642 95.4227) (width 0.25) (layer F.Cu) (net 10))
 (segment (start 178.642 95.4227) (end 177.719 94.5001) (width 0.25) (layer F.Cu) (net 10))
 (segment (start 177.719 94.5001) (end 177.719 93.98) (width 0.25) (layer F.Cu) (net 10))
 (segment (start 177.719 93.98) (end 176.53 93.98) (width 0.25) (layer F.Cu) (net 10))
 (segment (start 184.5 122) (end 182.17 119.67) (width 1) (layer F.Cu) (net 1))
 (segment (start 182.17 119.67) (end 173.83 119.67) (width 1) (layer F.Cu) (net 1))
 (segment (start 173.83 119.67) (end 171.5 122) (width 1) (layer F.Cu) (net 1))
 (segment (start 171.5 122) (end 168.601 119.101) (width 1) (layer F.Cu) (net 1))
 (segment (start 168.601 119.101) (end 151.744 119.101) (width 1) (layer F.Cu) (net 1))
 (segment (start 151.744 119.101) (end 150.5 117.856) (width 1) (layer F.Cu) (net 1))
 (segment (start 150.5 117.856) (end 150.5 116.04) (width 1) (layer F.Cu) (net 1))
 (segment (start 137 91.96) (end 135.336 91.96) (width 1) (layer B.Cu) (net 16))
 (segment (start 135.336 91.96) (end 135.336 96.8761) (width 1) (layer B.Cu) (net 16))
 (segment (start 135.336 96.8761) (end 138.46 100) (width 1) (layer B.Cu) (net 16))
 (segment (start 139.54 91.96) (end 137 91.96) (width 1) (layer F.Cu) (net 16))
 (segment (start 149.7 91.96) (end 150.889 91.96) (width 0.25) (layer B.Cu) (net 19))
 (segment (start 150.889 91.96) (end 150.889 91.4399) (width 0.25) (layer B.Cu) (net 19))
 (segment (start 150.889 91.4399) (end 151.662 90.6665) (width 0.25) (layer B.Cu) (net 19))
 (segment (start 151.662 90.6665) (end 155.214 90.6665) (width 0.25) (layer B.Cu) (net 19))
 (segment (start 155.214 90.6665) (end 155.979 91.4322) (width 0.25) (layer B.Cu) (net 19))
 (segment (start 155.979 91.4322) (end 155.979 95.013) (width 0.25) (layer B.Cu) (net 19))
 (segment (start 155.979 95.013) (end 175.638 114.672) (width 0.25) (layer B.Cu) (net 19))
 (segment (start 175.638 114.672) (end 178.286 114.672) (width 0.25) (layer B.Cu) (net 19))
 (segment (start 178.286 114.672) (end 181.817 118.203) (width 0.25) (layer B.Cu) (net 19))
 (segment (start 181.817 118.203) (end 187.837 118.203) (width 0.25) (layer B.Cu) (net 19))
 (segment (start 187.837 118.203) (end 189.54 116.5) (width 0.25) (layer B.Cu) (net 19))
 (segment (start 189 113.5) (end 189 114.675) (width 0.25) (layer F.Cu) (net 19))
 (segment (start 189 114.675) (end 189.229 114.905) (width 0.25) (layer F.Cu) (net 19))
 (segment (start 189.229 114.905) (end 189.54 114.905) (width 0.25) (layer F.Cu) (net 19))
 (segment (start 189.54 114.905) (end 189.54 116.5) (width 0.25) (layer F.Cu) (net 19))
 (segment (start 163.54 116.5) (end 163.54 114.905) (width 0.25) (layer F.Cu) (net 15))
 (segment (start 163.54 114.905) (end 163.229 114.905) (width 0.25) (layer F.Cu) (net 15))
 (segment (start 163.229 114.905) (end 163 114.675) (width 0.25) (layer F.Cu) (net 15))
 (segment (start 163 114.675) (end 163 113.5) (width 0.25) (layer F.Cu) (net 15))
 (segment (start 154.78 91.96) (end 154.78 93.1489) (width 0.25) (layer B.Cu) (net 15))
 (segment (start 154.78 93.1489) (end 154.408 93.1489) (width 0.25) (layer B.Cu) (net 15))
 (segment (start 154.408 93.1489) (end 153.565 93.9923) (width 0.25) (layer B.Cu) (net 15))
 (segment (start 153.565 93.9923) (end 153.565 95.051) (width 0.25) (layer B.Cu) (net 15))
 (segment (start 153.565 95.051) (end 163.54 105.026) (width 0.25) (layer B.Cu) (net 15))
 (segment (start 163.54 105.026) (end 163.54 116.5) (width 0.25) (layer B.Cu) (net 15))
 (segment (start 157.32 91.96) (end 158.509 91.96) (width 0.25) (layer F.Cu) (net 13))
 (segment (start 158.509 91.96) (end 158.509 92.4801) (width 0.25) (layer F.Cu) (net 13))
 (segment (start 158.509 92.4801) (end 159.33 93.3007) (width 0.25) (layer F.Cu) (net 13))
 (segment (start 159.33 93.3007) (end 160.347 93.3007) (width 0.25) (layer F.Cu) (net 13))
 (segment (start 160.347 93.3007) (end 161.13 94.0833) (width 0.25) (layer F.Cu) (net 13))
 (segment (start 161.13 94.0833) (end 161.13 94.972) (width 0.25) (layer F.Cu) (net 13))
 (segment (start 161.13 94.972) (end 164.256 98.0984) (width 0.25) (layer F.Cu) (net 13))
 (segment (start 164.256 98.0984) (end 178.621 98.0984) (width 0.25) (layer F.Cu) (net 13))
 (segment (start 178.621 98.0984) (end 180.826 100.304) (width 0.25) (layer F.Cu) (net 13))
 (segment (start 180.826 100.304) (end 180.826 109.999) (width 0.25) (layer F.Cu) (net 13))
 (segment (start 180.826 109.999) (end 177.325 113.5) (width 0.25) (layer F.Cu) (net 13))
 (segment (start 177.325 113.5) (end 176 113.5) (width 0.25) (layer F.Cu) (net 13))
 (segment (start 176.54 116.5) (end 176.54 114.905) (width 0.25) (layer F.Cu) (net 13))
 (segment (start 176.54 114.905) (end 176.229 114.905) (width 0.25) (layer F.Cu) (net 13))
 (segment (start 176.229 114.905) (end 176 114.675) (width 0.25) (layer F.Cu) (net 13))
 (segment (start 176 114.675) (end 176 113.5) (width 0.25) (layer F.Cu) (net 13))
 (segment (start 164.94 91.96) (end 164.94 94.5) (width 0.25) (layer F.Cu) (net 25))
 (segment (start 144.62 91.96) (end 145.809 91.96) (width 0.25) (layer F.Cu) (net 8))
 (segment (start 145.809 91.96) (end 145.809 92.3316) (width 0.25) (layer F.Cu) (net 8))
 (segment (start 145.809 92.3316) (end 146.626 93.1489) (width 0.25) (layer F.Cu) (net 8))
 (segment (start 146.626 93.1489) (end 149.166 93.1489) (width 0.25) (layer F.Cu) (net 8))
 (segment (start 149.166 93.1489) (end 149.266 93.249) (width 0.25) (layer F.Cu) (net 8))
 (segment (start 149.266 93.249) (end 154.536 93.249) (width 0.25) (layer F.Cu) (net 8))
 (segment (start 154.536 93.249) (end 154.625 93.1593) (width 0.25) (layer F.Cu) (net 8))
 (segment (start 154.625 93.1593) (end 157.846 93.1593) (width 0.25) (layer F.Cu) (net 8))
 (segment (start 157.846 93.1593) (end 158.661 93.9744) (width 0.25) (layer F.Cu) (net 8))
 (segment (start 158.661 93.9744) (end 158.661 94.983) (width 0.25) (layer F.Cu) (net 8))
 (segment (start 158.661 94.983) (end 165.773 102.095) (width 0.25) (layer F.Cu) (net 8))
 (segment (start 165.773 102.095) (end 177.11 102.095) (width 0.25) (layer F.Cu) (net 8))
 (segment (start 163.5 122) (end 161 119.5) (width 1) (layer B.Cu) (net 14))
 (segment (start 161 119.5) (end 161 116.5) (width 1) (layer B.Cu) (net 14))
 (segment (start 147.16 91.96) (end 147.16 93.1489) (width 0.25) (layer B.Cu) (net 7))
 (segment (start 147.16 93.1489) (end 147.68 93.1489) (width 0.25) (layer B.Cu) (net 7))
 (segment (start 147.68 93.1489) (end 148.501 93.9695) (width 0.25) (layer B.Cu) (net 7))
 (segment (start 148.501 93.9695) (end 148.501 95.0261) (width 0.25) (layer B.Cu) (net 7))
 (segment (start 148.501 95.0261) (end 149.735 96.26) (width 0.25) (layer B.Cu) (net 7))
 (segment (start 149.735 96.26) (end 153.494 96.26) (width 0.25) (layer B.Cu) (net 7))
 (segment (start 153.494 96.26) (end 155.709 98.4751) (width 0.25) (layer B.Cu) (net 7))
 (segment (start 155.709 98.4751) (end 159.52 98.4751) (width 0.25) (layer F.Cu) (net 7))
 (segment (start 159.52 98.4751) (end 164.41 103.365) (width 0.25) (layer F.Cu) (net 7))
 (segment (start 164.41 103.365) (end 179.65 103.365) (width 0.25) (layer F.Cu) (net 7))
 (via (at 155.709 98.4751) (size 0.6) (layers F.Cu B.Cu) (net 7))
 (segment (start 174 116.5) (end 174 119.5) (width 1) (layer B.Cu) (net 12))
 (segment (start 174 119.5) (end 176.5 122) (width 1) (layer B.Cu) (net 12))
 (segment (start 187 116.5) (end 187 119.5) (width 1) (layer F.Cu) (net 2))
 (segment (start 187 119.5) (end 189.5 122) (width 1) (layer F.Cu) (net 2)))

